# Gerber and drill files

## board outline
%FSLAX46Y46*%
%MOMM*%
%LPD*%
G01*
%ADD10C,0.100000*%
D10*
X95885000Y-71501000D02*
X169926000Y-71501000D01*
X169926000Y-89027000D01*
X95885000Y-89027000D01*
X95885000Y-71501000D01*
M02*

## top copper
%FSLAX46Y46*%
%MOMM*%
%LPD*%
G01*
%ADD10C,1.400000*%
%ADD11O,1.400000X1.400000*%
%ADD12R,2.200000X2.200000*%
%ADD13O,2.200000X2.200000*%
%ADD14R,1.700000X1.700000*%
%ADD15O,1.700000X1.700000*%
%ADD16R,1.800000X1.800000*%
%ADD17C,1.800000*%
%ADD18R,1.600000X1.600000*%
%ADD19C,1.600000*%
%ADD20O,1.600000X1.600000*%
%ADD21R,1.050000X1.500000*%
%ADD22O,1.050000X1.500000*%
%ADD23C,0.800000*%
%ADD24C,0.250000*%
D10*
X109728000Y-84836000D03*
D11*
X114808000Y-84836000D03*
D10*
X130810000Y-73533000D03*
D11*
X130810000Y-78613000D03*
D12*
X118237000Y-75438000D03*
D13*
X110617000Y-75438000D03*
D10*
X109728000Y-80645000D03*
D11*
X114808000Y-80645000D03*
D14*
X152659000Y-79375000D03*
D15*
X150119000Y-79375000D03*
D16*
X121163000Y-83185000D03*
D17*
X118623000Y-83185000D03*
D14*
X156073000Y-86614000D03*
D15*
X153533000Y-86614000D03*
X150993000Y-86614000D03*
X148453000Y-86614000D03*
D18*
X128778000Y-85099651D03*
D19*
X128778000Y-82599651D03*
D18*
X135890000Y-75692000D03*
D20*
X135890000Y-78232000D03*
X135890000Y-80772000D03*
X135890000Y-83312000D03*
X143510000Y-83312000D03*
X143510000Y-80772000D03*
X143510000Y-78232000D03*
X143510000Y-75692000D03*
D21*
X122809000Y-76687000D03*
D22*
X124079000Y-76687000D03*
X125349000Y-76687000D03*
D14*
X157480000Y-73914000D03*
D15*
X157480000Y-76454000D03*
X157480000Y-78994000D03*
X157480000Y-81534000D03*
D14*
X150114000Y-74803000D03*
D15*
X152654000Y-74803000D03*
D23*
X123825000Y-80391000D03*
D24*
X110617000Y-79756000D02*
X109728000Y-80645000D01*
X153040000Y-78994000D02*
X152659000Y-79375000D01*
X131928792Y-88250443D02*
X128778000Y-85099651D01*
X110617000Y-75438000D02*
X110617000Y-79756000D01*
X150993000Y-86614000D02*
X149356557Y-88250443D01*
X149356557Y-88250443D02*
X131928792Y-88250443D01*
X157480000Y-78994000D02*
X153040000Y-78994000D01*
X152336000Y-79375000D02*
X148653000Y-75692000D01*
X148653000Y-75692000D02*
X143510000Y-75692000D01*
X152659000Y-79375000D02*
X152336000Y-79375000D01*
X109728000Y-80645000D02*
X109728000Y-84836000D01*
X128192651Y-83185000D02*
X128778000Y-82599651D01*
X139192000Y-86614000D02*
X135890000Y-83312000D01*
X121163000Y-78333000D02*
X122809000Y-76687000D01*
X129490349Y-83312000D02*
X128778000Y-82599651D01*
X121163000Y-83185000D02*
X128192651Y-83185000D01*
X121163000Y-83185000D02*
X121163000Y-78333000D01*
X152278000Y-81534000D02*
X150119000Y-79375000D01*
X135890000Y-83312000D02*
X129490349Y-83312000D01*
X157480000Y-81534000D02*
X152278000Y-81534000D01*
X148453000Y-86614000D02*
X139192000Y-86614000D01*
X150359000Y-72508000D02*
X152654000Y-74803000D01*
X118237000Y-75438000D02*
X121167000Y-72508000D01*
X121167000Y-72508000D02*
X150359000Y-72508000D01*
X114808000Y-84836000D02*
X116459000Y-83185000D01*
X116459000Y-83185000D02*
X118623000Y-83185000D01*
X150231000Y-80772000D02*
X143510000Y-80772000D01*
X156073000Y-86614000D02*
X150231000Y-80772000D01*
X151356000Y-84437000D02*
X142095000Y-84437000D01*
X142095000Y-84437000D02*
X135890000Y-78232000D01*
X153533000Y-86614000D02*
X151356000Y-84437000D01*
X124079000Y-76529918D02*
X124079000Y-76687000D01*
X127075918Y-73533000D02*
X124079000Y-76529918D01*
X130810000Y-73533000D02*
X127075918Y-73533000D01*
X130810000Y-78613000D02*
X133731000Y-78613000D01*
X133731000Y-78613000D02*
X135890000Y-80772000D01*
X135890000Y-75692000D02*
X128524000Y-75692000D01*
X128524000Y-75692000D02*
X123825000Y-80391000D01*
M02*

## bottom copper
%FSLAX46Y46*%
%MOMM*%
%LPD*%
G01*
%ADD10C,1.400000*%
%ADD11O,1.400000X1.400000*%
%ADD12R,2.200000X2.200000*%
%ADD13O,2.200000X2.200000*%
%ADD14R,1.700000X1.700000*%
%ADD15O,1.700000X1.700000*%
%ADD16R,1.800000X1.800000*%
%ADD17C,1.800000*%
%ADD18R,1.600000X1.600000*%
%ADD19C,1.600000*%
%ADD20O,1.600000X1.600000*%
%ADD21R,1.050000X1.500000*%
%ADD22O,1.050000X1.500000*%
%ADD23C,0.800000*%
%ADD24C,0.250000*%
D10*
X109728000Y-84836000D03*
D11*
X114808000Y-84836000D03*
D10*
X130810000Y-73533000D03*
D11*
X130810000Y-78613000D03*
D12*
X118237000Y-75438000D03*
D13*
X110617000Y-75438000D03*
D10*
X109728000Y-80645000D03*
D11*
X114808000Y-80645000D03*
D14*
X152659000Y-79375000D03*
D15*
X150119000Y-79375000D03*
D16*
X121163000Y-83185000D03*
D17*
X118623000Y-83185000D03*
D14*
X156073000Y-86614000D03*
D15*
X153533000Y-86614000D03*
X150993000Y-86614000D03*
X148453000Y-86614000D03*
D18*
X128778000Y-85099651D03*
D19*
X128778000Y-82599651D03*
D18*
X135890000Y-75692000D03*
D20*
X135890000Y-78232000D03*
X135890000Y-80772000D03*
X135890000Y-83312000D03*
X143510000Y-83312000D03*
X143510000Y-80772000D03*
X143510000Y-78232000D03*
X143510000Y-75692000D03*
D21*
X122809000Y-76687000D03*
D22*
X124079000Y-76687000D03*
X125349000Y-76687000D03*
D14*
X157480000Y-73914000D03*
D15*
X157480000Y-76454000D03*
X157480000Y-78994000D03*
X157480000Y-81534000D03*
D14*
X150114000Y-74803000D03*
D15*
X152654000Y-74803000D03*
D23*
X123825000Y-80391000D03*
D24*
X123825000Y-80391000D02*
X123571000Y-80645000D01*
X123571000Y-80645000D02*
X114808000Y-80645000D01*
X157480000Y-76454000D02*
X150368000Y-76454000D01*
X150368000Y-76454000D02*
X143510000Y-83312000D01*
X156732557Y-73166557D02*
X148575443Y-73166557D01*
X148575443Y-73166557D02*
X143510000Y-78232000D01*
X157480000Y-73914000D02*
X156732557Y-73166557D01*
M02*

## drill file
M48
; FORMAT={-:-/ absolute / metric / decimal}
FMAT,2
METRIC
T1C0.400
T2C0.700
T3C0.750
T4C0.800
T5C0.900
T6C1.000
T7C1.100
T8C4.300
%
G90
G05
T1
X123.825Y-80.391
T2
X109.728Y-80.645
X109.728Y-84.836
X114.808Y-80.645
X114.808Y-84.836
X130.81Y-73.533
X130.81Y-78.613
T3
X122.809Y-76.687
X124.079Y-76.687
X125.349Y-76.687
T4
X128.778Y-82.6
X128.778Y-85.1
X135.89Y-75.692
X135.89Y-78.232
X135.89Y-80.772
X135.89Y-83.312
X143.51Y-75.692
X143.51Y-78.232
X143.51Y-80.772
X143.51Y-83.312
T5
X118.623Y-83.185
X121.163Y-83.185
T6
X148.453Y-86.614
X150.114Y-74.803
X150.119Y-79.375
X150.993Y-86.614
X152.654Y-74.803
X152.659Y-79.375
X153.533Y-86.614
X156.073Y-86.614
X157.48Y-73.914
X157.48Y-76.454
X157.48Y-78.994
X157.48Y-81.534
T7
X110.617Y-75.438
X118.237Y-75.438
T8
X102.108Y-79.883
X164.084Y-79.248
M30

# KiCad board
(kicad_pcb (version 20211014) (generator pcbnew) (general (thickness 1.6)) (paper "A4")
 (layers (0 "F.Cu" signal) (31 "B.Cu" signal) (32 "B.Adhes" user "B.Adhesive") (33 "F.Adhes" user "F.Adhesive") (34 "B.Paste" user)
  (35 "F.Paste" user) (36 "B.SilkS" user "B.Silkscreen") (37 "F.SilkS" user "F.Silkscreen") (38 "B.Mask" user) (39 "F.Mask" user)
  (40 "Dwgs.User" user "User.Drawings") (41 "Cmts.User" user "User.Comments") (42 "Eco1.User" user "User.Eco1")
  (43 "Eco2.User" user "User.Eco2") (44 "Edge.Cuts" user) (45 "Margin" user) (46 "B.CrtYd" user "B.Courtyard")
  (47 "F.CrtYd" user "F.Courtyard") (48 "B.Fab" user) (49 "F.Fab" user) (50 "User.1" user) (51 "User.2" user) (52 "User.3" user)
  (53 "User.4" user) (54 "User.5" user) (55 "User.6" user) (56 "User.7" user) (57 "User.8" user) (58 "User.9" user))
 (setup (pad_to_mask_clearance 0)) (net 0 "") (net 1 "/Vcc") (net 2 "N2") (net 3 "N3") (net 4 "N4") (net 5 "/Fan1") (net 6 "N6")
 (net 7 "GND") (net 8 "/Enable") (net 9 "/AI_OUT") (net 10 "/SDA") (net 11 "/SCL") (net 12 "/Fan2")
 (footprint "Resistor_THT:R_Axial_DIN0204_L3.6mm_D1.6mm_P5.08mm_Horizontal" (layer "F.Cu") (at 109.728 84.836)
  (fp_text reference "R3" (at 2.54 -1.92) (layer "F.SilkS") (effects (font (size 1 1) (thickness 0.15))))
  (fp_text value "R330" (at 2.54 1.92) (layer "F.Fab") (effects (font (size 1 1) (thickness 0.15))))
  (pad "1" thru_hole circle (at 0 0) (size 1.4 1.4) (drill 0.7) (layers *.Cu *.Mask) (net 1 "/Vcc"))
  (pad "2" thru_hole oval (at 5.08 0) (size 1.4 1.4) (drill 0.7) (layers *.Cu *.Mask) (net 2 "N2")))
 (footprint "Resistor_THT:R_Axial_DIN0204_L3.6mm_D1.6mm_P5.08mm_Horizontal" (layer "F.Cu") (at 130.81 73.533 -90)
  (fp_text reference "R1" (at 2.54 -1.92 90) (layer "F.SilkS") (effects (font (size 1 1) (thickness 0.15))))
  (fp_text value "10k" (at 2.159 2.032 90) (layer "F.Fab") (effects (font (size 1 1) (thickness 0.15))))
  (pad "1" thru_hole circle (at 0 0 270) (size 1.4 1.4) (drill 0.7) (layers *.Cu *.Mask) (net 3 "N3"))
  (pad "2" thru_hole oval (at 5.08 0 270) (size 1.4 1.4) (drill 0.7) (layers *.Cu *.Mask) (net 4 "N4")))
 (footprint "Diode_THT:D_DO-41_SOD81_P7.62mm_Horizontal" (layer "F.Cu") (at 118.237 75.438 180)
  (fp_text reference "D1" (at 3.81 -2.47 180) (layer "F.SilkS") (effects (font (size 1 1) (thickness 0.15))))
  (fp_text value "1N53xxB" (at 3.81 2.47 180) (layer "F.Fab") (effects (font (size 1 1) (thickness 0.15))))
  (pad "1" thru_hole rect (at 0 0 180) (size 2.2 2.2) (drill 1.1) (layers *.Cu *.Mask) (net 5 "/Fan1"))
  (pad "2" thru_hole oval (at 7.62 0 180) (size 2.2 2.2) (drill 1.1) (layers *.Cu *.Mask) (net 1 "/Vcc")))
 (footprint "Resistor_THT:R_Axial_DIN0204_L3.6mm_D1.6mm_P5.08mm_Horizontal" (layer "F.Cu") (at 109.728 80.645)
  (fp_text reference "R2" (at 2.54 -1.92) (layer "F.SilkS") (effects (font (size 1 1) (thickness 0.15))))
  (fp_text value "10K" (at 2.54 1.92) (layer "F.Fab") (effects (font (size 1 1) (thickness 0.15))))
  (pad "1" thru_hole circle (at 0 0) (size 1.4 1.4) (drill 0.7) (layers *.Cu *.Mask) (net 1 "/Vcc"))
  (pad "2" thru_hole oval (at 5.08 0) (size 1.4 1.4) (drill 0.7) (layers *.Cu *.Mask) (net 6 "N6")))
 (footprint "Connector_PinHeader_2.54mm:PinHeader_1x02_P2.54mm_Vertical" (layer "F.Cu") (at 152.659 79.375 -90)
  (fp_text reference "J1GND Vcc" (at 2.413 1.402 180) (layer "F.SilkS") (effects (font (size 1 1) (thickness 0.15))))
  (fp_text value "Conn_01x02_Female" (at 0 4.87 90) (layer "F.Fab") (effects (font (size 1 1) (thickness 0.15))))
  (pad "1" thru_hole rect (at 0 0 270) (size 1.7 1.7) (drill 1) (layers *.Cu *.Mask) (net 1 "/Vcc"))
  (pad "2" thru_hole oval (at 0 2.54 270) (size 1.7 1.7) (drill 1) (layers *.Cu *.Mask) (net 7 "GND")))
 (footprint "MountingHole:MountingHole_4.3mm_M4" (layer "F.Cu") (at 102.108 79.883)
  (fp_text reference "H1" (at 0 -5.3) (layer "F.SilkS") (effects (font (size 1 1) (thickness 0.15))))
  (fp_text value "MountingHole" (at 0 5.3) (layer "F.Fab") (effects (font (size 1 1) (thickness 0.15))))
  (pad "" np_thru_hole circle (at 0 0) (size 4.3 4.3) (drill 4.3) (layers *.Cu *.Mask)))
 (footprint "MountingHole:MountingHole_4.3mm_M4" (layer "F.Cu") (at 164.084 79.248)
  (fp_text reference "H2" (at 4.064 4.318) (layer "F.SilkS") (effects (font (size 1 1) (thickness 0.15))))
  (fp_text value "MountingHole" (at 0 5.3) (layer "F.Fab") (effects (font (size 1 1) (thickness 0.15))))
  (pad "" np_thru_hole circle (at 0 0) (size 4.3 4.3) (drill 4.3) (layers *.Cu *.Mask)))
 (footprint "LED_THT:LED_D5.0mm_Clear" (layer "F.Cu") (at 121.163 83.185 180)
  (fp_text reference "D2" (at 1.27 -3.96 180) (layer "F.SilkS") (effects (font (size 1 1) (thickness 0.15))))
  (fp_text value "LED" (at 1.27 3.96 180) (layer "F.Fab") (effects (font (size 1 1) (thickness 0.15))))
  (pad "1" thru_hole rect (at 0 0 180) (size 1.8 1.8) (drill 0.9) (layers *.Cu *.Mask) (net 7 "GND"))
  (pad "2" thru_hole circle (at 2.54 0 180) (size 1.8 1.8) (drill 0.9) (layers *.Cu *.Mask) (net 2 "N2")))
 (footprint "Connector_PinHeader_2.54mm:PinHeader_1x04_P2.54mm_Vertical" (layer "F.Cu") (at 156.073 86.614 -90)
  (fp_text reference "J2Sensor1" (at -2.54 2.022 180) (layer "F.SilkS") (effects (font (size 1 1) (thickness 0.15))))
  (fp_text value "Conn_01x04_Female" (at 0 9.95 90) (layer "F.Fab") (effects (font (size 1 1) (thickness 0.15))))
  (pad "1" thru_hole rect (at 0 0 270) (size 1.7 1.7) (drill 1) (layers *.Cu *.Mask) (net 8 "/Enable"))
  (pad "2" thru_hole oval (at 0 2.54 270) (size 1.7 1.7) (drill 1) (layers *.Cu *.Mask) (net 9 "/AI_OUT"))
  (pad "3" thru_hole oval (at 0 5.08 270) (size 1.7 1.7) (drill 1) (layers *.Cu *.Mask) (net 1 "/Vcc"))
  (pad "4" thru_hole oval (at 0 7.62 270) (size 1.7 1.7) (drill 1) (layers *.Cu *.Mask) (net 7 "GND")))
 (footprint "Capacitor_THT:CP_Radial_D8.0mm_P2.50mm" (layer "F.Cu") (at 128.778 85.099651 90)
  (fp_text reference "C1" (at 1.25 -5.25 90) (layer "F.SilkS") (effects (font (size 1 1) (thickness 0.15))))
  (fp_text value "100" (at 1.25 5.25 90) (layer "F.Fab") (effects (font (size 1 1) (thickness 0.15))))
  (pad "1" thru_hole rect (at 0 0 90) (size 1.6 1.6) (drill 0.8) (layers *.Cu *.Mask) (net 1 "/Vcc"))
  (pad "2" thru_hole circle (at 2.5 0 90) (size 1.6 1.6) (drill 0.8) (layers *.Cu *.Mask) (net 7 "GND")))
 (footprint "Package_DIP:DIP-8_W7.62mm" (layer "F.Cu") (at 135.89 75.692)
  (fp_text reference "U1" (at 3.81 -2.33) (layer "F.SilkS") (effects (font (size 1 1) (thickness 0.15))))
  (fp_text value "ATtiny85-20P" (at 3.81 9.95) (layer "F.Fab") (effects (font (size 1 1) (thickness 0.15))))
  (pad "1" thru_hole rect (at 0 0) (size 1.6 1.6) (drill 0.8) (layers *.Cu *.Mask) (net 6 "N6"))
  (pad "2" thru_hole oval (at 0 2.54) (size 1.6 1.6) (drill 0.8) (layers *.Cu *.Mask) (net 9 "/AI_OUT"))
  (pad "3" thru_hole oval (at 0 5.08) (size 1.6 1.6) (drill 0.8) (layers *.Cu *.Mask) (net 4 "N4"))
  (pad "4" thru_hole oval (at 0 7.62) (size 1.6 1.6) (drill 0.8) (layers *.Cu *.Mask) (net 7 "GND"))
  (pad "5" thru_hole oval (at 7.62 7.62) (size 1.6 1.6) (drill 0.8) (layers *.Cu *.Mask) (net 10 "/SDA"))
  (pad "6" thru_hole oval (at 7.62 5.08) (size 1.6 1.6) (drill 0.8) (layers *.Cu *.Mask) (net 8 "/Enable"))
  (pad "7" thru_hole oval (at 7.62 2.54) (size 1.6 1.6) (drill 0.8) (layers *.Cu *.Mask) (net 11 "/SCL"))
  (pad "8" thru_hole oval (at 7.62 0) (size 1.6 1.6) (drill 0.8) (layers *.Cu *.Mask) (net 1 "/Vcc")))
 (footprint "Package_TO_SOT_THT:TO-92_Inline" (layer "F.Cu") (at 122.809 76.687)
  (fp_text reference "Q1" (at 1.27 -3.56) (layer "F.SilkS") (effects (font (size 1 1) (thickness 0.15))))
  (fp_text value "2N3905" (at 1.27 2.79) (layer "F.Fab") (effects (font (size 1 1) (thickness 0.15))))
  (pad "1" thru_hole rect (at 0 0) (size 1.05 1.5) (drill 0.75) (layers *.Cu *.Mask) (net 7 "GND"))
  (pad "2" thru_hole oval (at 1.27 0) (size 1.05 1.5) (drill 0.75) (layers *.Cu *.Mask) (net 3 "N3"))
  (pad "3" thru_hole oval (at 2.54 0) (size 1.05 1.5) (drill 0.75) (layers *.Cu *.Mask) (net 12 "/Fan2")))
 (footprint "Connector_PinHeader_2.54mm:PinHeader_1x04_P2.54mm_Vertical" (layer "F.Cu") (at 157.48 73.914)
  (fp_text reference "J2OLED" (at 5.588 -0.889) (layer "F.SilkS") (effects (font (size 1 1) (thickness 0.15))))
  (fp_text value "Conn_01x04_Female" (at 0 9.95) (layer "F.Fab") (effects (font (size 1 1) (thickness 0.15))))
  (pad "1" thru_hole rect (at 0 0) (size 1.7 1.7) (drill 1) (layers *.Cu *.Mask) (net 11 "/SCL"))
  (pad "2" thru_hole oval (at 0 2.54) (size 1.7 1.7) (drill 1) (layers *.Cu *.Mask) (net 10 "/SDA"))
  (pad "3" thru_hole oval (at 0 5.08) (size 1.7 1.7) (drill 1) (layers *.Cu *.Mask) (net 1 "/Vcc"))
  (pad "4" thru_hole oval (at 0 7.62) (size 1.7 1.7) (drill 1) (layers *.Cu *.Mask) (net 7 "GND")))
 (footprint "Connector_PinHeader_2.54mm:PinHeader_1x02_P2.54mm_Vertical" (layer "F.Cu") (at 150.114 74.803 90)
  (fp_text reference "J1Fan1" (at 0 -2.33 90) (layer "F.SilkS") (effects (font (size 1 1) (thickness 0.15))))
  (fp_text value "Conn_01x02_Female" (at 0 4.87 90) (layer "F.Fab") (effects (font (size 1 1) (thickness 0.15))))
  (pad "1" thru_hole rect (at 0 0 90) (size 1.7 1.7) (drill 1) (layers *.Cu *.Mask) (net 12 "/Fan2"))
  (pad "2" thru_hole oval (at 0 2.54 90) (size 1.7 1.7) (drill 1) (layers *.Cu *.Mask) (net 5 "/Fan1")))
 (gr_rect (start 95.885 71.501) (end 169.926 89.027) (layer "Edge.Cuts") (width 0.1) (fill none))
 (segment (start 110.617 79.756) (end 109.728 80.645) (width 0.25) (layer "F.Cu") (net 1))
 (segment (start 153.04 78.994) (end 152.659 79.375) (width 0.25) (layer "F.Cu") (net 1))
 (segment (start 131.928792 88.250443) (end 128.778 85.099651) (width 0.25) (layer "F.Cu") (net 1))
 (segment (start 110.617 75.438) (end 110.617 79.756) (width 0.25) (layer "F.Cu") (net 1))
 (segment (start 150.993 86.614) (end 149.356557 88.250443) (width 0.25) (layer "F.Cu") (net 1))
 (segment (start 149.356557 88.250443) (end 131.928792 88.250443) (width 0.25) (layer "F.Cu") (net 1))
 (segment (start 157.48 78.994) (end 153.04 78.994) (width 0.25) (layer "F.Cu") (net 1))
 (segment (start 152.336 79.375) (end 148.653 75.692) (width 0.25) (layer "F.Cu") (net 1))
 (segment (start 148.653 75.692) (end 143.51 75.692) (width 0.25) (layer "F.Cu") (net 1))
 (segment (start 152.659 79.375) (end 152.336 79.375) (width 0.25) (layer "F.Cu") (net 1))
 (segment (start 109.728 80.645) (end 109.728 84.836) (width 0.25) (layer "F.Cu") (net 1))
 (segment (start 128.192651 83.185) (end 128.778 82.599651) (width 0.25) (layer "F.Cu") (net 7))
 (segment (start 139.192 86.614) (end 135.89 83.312) (width 0.25) (layer "F.Cu") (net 7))
 (segment (start 121.163 78.333) (end 122.809 76.687) (width 0.25) (layer "F.Cu") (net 7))
 (segment (start 129.490349 83.312) (end 128.778 82.599651) (width 0.25) (layer "F.Cu") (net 7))
 (segment (start 121.163 83.185) (end 128.192651 83.185) (width 0.25) (layer "F.Cu") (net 7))
 (segment (start 121.163 83.185) (end 121.163 78.333) (width 0.25) (layer "F.Cu") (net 7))
 (segment (start 152.278 81.534) (end 150.119 79.375) (width 0.25) (layer "F.Cu") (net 7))
 (segment (start 135.89 83.312) (end 129.490349 83.312) (width 0.25) (layer "F.Cu") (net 7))
 (segment (start 157.48 81.534) (end 152.278 81.534) (width 0.25) (layer "F.Cu") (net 7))
 (segment (start 148.453 86.614) (end 139.192 86.614) (width 0.25) (layer "F.Cu") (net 7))
 (segment (start 150.359 72.508) (end 152.654 74.803) (width 0.25) (layer "F.Cu") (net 5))
 (segment (start 118.237 75.438) (end 121.167 72.508) (width 0.25) (layer "F.Cu") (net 5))
 (segment (start 121.167 72.508) (end 150.359 72.508) (width 0.25) (layer "F.Cu") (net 5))
 (segment (start 114.808 84.836) (end 116.459 83.185) (width 0.25) (layer "F.Cu") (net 2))
 (segment (start 116.459 83.185) (end 118.623 83.185) (width 0.25) (layer "F.Cu") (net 2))
 (segment (start 150.231 80.772) (end 143.51 80.772) (width 0.25) (layer "F.Cu") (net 8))
 (segment (start 156.073 86.614) (end 150.231 80.772) (width 0.25) (layer "F.Cu") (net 8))
 (segment (start 151.356 84.437) (end 142.095 84.437) (width 0.25) (layer "F.Cu") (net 9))
 (segment (start 142.095 84.437) (end 135.89 78.232) (width 0.25) (layer "F.Cu") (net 9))
 (segment (start 153.533 86.614) (end 151.356 84.437) (width 0.25) (layer "F.Cu") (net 9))
 (segment (start 124.079 76.529918) (end 124.079 76.687) (width 0.25) (layer "F.Cu") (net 3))
 (segment (start 127.075918 73.533) (end 124.079 76.529918) (width 0.25) (layer "F.Cu") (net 3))
 (segment (start 130.81 73.533) (end 127.075918 73.533) (width 0.25) (layer "F.Cu") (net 3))
 (segment (start 130.81 78.613) (end 133.731 78.613) (width 0.25) (layer "F.Cu") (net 4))
 (segment (start 133.731 78.613) (end 135.89 80.772) (width 0.25) (layer "F.Cu") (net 4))
 (segment (start 135.89 75.692) (end 128.524 75.692) (width 0.25) (layer "F.Cu") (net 6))
 (segment (start 128.524 75.692) (end 123.825 80.391) (width 0.25) (layer "F.Cu") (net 6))
 (via (at 123.825 80.391) (size 0.8) (drill 0.4) (layers "F.Cu" "B.Cu") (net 6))
 (segment (start 123.825 80.391) (end 123.571 80.645) (width 0.25) (layer "B.Cu") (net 6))
 (segment (start 123.571 80.645) (end 114.808 80.645) (width 0.25) (layer "B.Cu") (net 6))
 (segment (start 157.48 76.454) (end 150.368 76.454) (width 0.25) (layer "B.Cu") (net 10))
 (segment (start 150.368 76.454) (end 143.51 83.312) (width 0.25) (layer "B.Cu") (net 10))
 (segment (start 156.732557 73.166557) (end 148.575443 73.166557) (width 0.25) (layer "B.Cu") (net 11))
 (segment (start 148.575443 73.166557) (end 143.51 78.232) (width 0.25) (layer "B.Cu") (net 11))
 (segment (start 157.48 73.914) (end 156.732557 73.166557) (width 0.25) (layer "B.Cu") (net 11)))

